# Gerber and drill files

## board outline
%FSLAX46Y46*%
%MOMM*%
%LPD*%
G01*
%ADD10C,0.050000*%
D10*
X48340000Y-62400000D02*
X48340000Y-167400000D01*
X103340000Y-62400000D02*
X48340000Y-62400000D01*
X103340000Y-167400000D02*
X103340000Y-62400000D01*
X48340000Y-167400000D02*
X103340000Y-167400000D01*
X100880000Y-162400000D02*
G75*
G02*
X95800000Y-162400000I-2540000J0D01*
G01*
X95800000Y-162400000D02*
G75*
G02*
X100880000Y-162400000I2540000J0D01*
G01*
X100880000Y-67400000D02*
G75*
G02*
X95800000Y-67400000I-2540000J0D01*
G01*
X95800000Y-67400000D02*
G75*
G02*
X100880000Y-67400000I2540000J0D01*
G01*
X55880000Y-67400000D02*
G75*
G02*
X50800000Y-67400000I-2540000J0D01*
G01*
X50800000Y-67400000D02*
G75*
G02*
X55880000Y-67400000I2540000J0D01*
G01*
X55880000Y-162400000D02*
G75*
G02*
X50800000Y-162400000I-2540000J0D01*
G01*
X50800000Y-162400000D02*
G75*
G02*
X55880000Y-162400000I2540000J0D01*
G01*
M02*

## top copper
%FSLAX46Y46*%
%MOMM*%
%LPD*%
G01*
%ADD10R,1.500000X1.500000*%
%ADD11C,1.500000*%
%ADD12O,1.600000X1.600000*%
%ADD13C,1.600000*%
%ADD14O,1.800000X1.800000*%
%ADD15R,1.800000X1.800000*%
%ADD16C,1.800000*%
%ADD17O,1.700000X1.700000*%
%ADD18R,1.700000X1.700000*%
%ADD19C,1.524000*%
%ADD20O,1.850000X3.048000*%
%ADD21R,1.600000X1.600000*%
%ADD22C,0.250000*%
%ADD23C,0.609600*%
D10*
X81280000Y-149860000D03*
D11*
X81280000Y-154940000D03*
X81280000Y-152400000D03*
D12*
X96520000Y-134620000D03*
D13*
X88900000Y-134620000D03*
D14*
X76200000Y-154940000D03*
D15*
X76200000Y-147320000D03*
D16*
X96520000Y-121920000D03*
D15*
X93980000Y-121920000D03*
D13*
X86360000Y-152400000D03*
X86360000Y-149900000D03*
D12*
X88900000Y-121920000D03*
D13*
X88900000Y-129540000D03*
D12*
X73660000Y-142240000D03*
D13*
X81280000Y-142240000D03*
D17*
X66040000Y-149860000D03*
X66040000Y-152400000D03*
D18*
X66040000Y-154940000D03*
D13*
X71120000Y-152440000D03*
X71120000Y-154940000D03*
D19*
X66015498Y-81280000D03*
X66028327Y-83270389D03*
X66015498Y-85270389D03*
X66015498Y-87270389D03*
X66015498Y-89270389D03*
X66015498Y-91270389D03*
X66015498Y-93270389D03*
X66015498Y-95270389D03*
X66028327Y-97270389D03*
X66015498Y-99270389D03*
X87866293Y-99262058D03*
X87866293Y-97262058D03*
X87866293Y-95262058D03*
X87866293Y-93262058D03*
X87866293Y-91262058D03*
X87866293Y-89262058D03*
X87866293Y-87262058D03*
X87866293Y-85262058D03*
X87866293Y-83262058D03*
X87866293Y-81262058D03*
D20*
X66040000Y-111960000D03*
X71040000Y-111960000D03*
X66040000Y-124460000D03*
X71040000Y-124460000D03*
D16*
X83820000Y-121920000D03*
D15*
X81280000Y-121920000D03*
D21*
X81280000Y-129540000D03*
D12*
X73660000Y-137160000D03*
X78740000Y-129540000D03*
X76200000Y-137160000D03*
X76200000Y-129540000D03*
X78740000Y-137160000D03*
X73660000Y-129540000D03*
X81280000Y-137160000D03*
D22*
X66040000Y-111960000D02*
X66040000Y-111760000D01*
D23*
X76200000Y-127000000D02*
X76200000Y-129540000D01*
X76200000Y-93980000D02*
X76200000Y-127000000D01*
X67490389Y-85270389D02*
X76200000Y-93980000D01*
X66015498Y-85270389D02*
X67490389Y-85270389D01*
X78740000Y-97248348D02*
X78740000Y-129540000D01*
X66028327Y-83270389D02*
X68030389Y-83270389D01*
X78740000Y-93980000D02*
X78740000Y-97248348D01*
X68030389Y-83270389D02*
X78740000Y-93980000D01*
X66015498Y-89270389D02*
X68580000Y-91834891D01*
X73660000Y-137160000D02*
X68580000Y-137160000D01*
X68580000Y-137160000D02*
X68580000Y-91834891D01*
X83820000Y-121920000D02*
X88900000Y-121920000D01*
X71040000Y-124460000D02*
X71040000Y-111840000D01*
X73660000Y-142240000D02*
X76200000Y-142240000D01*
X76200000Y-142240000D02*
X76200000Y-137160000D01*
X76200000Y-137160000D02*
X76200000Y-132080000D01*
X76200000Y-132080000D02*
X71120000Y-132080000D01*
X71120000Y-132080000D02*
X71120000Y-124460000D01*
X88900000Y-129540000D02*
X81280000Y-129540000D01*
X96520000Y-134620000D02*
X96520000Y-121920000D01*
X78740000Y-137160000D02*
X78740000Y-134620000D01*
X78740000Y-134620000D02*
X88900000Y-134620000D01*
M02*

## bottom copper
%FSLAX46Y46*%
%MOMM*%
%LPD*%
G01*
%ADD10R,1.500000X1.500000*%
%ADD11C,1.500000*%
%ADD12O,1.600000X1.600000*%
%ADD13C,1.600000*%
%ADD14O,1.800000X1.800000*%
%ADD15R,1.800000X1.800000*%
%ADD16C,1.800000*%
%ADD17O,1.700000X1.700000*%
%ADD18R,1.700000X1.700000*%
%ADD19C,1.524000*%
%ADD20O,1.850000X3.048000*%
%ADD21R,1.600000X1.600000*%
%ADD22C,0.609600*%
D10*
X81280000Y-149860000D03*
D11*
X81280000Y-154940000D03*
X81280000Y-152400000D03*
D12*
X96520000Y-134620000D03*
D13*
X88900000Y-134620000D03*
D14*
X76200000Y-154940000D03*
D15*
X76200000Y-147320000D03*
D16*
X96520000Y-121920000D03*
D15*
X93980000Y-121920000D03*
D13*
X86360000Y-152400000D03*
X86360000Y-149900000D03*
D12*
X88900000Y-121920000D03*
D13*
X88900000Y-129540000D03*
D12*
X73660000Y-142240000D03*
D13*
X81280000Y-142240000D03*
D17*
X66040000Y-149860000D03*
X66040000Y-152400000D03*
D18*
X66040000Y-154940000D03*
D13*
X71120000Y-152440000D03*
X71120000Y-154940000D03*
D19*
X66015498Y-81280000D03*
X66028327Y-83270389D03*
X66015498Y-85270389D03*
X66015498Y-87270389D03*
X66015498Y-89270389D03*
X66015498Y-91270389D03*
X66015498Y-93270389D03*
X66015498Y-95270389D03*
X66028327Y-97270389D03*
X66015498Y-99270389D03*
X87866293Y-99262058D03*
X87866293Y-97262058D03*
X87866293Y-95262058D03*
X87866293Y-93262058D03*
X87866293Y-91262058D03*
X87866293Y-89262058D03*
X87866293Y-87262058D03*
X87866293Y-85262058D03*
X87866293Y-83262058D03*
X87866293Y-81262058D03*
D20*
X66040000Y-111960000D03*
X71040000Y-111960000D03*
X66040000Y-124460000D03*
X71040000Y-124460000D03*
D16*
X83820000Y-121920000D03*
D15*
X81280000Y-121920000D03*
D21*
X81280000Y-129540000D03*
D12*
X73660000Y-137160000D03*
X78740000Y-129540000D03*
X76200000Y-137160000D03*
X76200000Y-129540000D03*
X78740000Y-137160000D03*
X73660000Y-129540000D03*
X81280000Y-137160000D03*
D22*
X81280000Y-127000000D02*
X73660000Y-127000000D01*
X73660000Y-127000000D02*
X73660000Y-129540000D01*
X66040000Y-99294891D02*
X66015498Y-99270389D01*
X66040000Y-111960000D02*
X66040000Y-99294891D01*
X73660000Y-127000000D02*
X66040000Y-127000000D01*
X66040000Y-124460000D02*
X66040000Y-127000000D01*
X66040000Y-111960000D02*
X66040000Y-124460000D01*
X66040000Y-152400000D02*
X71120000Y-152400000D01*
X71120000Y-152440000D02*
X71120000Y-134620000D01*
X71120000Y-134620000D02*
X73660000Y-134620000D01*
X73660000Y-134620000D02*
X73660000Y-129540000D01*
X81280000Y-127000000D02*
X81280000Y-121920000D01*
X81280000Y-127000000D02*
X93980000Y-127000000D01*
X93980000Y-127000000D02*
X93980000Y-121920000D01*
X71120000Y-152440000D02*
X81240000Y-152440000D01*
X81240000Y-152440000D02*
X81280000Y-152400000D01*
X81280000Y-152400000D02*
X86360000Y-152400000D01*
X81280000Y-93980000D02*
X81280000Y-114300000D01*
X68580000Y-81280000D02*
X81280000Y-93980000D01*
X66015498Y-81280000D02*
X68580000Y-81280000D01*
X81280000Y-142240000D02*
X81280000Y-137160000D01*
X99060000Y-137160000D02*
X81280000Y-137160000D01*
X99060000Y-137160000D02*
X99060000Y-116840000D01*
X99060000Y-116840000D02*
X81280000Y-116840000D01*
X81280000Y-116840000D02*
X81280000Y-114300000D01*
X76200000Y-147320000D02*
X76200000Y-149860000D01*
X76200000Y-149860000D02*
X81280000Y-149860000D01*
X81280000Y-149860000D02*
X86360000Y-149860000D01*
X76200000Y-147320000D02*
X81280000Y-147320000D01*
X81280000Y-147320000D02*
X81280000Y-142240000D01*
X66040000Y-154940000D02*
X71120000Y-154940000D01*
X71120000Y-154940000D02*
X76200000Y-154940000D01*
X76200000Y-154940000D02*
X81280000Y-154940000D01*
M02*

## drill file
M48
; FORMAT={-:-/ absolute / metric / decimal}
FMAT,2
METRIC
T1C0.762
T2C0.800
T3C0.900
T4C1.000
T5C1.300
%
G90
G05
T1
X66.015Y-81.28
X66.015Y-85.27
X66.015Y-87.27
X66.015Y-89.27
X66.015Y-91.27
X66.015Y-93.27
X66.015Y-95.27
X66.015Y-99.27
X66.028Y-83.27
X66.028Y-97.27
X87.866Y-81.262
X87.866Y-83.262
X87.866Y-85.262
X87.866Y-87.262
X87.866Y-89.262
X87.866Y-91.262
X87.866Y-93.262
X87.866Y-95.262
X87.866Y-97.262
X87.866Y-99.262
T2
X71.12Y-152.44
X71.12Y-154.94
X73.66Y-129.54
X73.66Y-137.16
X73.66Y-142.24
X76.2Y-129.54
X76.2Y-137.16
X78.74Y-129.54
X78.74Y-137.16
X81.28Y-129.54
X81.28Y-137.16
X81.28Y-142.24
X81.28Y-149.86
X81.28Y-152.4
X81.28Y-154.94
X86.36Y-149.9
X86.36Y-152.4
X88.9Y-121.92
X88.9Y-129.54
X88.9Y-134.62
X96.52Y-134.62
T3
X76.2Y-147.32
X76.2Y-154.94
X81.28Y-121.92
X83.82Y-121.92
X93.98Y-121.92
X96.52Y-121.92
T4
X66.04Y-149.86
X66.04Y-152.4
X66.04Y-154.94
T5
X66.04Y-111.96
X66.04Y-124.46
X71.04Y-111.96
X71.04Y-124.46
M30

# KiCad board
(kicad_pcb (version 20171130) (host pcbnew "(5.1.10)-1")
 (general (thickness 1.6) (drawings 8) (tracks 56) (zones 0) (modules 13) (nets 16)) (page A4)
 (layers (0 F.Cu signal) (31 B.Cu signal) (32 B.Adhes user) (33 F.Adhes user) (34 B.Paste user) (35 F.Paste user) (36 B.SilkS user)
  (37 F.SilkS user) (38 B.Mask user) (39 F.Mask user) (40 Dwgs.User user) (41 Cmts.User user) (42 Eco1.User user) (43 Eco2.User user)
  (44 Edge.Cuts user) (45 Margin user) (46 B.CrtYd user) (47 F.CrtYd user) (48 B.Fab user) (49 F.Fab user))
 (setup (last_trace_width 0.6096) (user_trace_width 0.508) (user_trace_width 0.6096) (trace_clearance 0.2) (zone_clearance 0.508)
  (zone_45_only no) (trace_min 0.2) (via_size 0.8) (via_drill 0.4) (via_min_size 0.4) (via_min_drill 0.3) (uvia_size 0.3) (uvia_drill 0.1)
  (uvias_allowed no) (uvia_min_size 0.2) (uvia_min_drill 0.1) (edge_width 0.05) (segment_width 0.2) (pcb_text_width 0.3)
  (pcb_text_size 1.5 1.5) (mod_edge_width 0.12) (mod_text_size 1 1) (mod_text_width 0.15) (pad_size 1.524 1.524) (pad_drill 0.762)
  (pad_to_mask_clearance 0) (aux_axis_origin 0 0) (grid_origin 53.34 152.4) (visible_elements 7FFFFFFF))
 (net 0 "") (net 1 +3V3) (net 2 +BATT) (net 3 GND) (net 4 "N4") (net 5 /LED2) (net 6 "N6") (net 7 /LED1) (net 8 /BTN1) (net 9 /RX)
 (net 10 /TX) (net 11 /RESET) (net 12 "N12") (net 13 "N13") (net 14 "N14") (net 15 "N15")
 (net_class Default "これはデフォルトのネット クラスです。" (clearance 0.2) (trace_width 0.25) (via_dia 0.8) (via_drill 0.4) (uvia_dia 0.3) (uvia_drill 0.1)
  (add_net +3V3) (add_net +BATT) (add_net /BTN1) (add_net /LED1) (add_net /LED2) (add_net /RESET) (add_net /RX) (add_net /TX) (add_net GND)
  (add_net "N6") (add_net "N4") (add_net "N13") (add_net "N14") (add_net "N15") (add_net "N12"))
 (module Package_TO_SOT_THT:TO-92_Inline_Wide (layer F.Cu) (at 81.28 149.86 270)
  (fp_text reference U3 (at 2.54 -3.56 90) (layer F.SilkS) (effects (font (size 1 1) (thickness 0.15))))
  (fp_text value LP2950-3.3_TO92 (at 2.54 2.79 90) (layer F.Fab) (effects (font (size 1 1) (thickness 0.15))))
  (pad 1 thru_hole rect (at 0 0 270) (size 1.5 1.5) (drill 0.8) (layers *.Cu *.Mask) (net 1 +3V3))
  (pad 3 thru_hole circle (at 5.08 0 270) (size 1.5 1.5) (drill 0.8) (layers *.Cu *.Mask) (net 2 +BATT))
  (pad 2 thru_hole circle (at 2.54 0 270) (size 1.5 1.5) (drill 0.8) (layers *.Cu *.Mask) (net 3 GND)))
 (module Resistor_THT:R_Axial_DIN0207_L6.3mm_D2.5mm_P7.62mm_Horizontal (layer F.Cu) (at 88.9 134.62)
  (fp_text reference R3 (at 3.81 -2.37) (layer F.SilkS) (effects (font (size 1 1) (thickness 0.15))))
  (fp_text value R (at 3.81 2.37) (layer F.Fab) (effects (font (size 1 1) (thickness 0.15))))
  (pad 2 thru_hole oval (at 7.62 0) (size 1.6 1.6) (drill 0.8) (layers *.Cu *.Mask) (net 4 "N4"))
  (pad 1 thru_hole circle (at 0 0) (size 1.6 1.6) (drill 0.8) (layers *.Cu *.Mask) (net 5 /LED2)))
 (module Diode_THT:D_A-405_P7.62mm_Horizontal (layer F.Cu) (at 76.2 147.32 270)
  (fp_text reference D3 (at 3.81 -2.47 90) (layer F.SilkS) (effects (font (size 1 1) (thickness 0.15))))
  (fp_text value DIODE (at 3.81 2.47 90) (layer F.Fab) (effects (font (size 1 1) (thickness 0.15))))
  (pad 2 thru_hole oval (at 7.62 0 270) (size 1.8 1.8) (drill 0.9) (layers *.Cu *.Mask) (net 2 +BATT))
  (pad 1 thru_hole rect (at 0 0 270) (size 1.8 1.8) (drill 0.9) (layers *.Cu *.Mask) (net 1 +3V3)))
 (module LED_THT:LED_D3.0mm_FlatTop (layer F.Cu) (at 93.98 121.92)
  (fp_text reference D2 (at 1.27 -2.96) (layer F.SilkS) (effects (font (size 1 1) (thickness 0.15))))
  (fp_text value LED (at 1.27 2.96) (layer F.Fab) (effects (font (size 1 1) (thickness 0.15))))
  (pad 2 thru_hole circle (at 2.54 0) (size 1.8 1.8) (drill 0.9) (layers *.Cu *.Mask) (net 4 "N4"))
  (pad 1 thru_hole rect (at 0 0) (size 1.8 1.8) (drill 0.9) (layers *.Cu *.Mask) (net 3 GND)))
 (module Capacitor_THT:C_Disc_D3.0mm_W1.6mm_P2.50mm (layer F.Cu) (at 86.36 149.9 270)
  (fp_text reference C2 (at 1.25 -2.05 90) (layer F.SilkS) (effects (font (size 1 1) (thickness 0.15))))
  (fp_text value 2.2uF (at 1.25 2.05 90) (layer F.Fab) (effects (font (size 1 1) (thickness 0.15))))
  (pad 2 thru_hole circle (at 2.5 0 270) (size 1.6 1.6) (drill 0.8) (layers *.Cu *.Mask) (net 3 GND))
  (pad 1 thru_hole circle (at 0 0 270) (size 1.6 1.6) (drill 0.8) (layers *.Cu *.Mask) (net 1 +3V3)))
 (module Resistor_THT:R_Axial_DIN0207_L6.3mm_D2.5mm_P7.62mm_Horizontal (layer F.Cu) (at 88.9 129.54 90)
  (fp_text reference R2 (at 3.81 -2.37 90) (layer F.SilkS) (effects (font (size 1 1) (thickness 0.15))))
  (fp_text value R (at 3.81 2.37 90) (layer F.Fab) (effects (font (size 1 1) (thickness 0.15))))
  (pad 2 thru_hole oval (at 7.62 0 90) (size 1.6 1.6) (drill 0.8) (layers *.Cu *.Mask) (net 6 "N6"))
  (pad 1 thru_hole circle (at 0 0 90) (size 1.6 1.6) (drill 0.8) (layers *.Cu *.Mask) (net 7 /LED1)))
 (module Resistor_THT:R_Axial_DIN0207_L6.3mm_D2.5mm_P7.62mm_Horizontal (layer F.Cu) (at 81.28 142.24 180)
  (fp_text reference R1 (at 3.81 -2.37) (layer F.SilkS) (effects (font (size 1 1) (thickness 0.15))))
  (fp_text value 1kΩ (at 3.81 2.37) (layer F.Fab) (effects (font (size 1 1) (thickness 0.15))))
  (pad 2 thru_hole oval (at 7.62 0 180) (size 1.6 1.6) (drill 0.8) (layers *.Cu *.Mask) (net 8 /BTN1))
  (pad 1 thru_hole circle (at 0 0 180) (size 1.6 1.6) (drill 0.8) (layers *.Cu *.Mask) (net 1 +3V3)))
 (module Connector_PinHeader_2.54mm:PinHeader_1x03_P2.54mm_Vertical (layer F.Cu) (at 66.04 154.94 180)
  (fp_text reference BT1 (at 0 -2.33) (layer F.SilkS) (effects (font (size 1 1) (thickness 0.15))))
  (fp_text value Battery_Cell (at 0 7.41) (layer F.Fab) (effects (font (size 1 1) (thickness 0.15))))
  (pad 3 thru_hole oval (at 0 5.08 180) (size 1.7 1.7) (drill 1) (layers *.Cu *.Mask))
  (pad 2 thru_hole oval (at 0 2.54 180) (size 1.7 1.7) (drill 1) (layers *.Cu *.Mask) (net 3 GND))
  (pad 1 thru_hole rect (at 0 0 180) (size 1.7 1.7) (drill 1) (layers *.Cu *.Mask) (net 2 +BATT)))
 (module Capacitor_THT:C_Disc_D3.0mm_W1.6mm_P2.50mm (layer F.Cu) (at 71.12 154.94 90)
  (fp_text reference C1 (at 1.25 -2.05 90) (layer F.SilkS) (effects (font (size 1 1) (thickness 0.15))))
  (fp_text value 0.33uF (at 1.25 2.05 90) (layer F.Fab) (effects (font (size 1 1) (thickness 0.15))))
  (pad 2 thru_hole circle (at 2.5 0 90) (size 1.6 1.6) (drill 0.8) (layers *.Cu *.Mask) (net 3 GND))
  (pad 1 thru_hole circle (at 0 0 90) (size 1.6 1.6) (drill 0.8) (layers *.Cu *.Mask) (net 2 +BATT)))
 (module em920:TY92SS (layer F.Cu) (at 64.77 107.929212)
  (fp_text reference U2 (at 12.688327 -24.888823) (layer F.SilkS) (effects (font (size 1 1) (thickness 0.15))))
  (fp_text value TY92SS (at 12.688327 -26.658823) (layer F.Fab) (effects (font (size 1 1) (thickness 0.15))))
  (pad 1 thru_hole circle (at 1.245498 -26.649212) (size 1.524 1.524) (drill 0.762) (layers *.Cu *.Mask) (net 1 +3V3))
  (pad 2 thru_hole circle (at 1.258327 -24.658823) (size 1.524 1.524) (drill 0.762) (layers *.Cu *.Mask) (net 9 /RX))
  (pad 3 thru_hole circle (at 1.245498 -22.658823) (size 1.524 1.524) (drill 0.762) (layers *.Cu *.Mask) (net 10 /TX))
  (pad 4 thru_hole circle (at 1.245498 -20.658823) (size 1.524 1.524) (drill 0.762) (layers *.Cu *.Mask))
  (pad 5 thru_hole circle (at 1.245498 -18.658823) (size 1.524 1.524) (drill 0.762) (layers *.Cu *.Mask) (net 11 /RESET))
  (pad 6 thru_hole circle (at 1.245498 -16.658823) (size 1.524 1.524) (drill 0.762) (layers *.Cu *.Mask))
  (pad 7 thru_hole circle (at 1.245498 -14.658823) (size 1.524 1.524) (drill 0.762) (layers *.Cu *.Mask))
  (pad 8 thru_hole circle (at 1.245498 -12.658823) (size 1.524 1.524) (drill 0.762) (layers *.Cu *.Mask))
  (pad 9 thru_hole circle (at 1.258327 -10.658823) (size 1.524 1.524) (drill 0.762) (layers *.Cu *.Mask) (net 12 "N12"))
  (pad 10 thru_hole circle (at 1.245498 -8.658823) (size 1.524 1.524) (drill 0.762) (layers *.Cu *.Mask) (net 3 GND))
  (pad 11 thru_hole circle (at 23.096293 -8.667154) (size 1.524 1.524) (drill 0.762) (layers *.Cu *.Mask))
  (pad 12 thru_hole circle (at 23.096293 -10.667154) (size 1.524 1.524) (drill 0.762) (layers *.Cu *.Mask) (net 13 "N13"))
  (pad 13 thru_hole circle (at 23.096293 -12.667154) (size 1.524 1.524) (drill 0.762) (layers *.Cu *.Mask) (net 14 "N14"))
  (pad 14 thru_hole circle (at 23.096293 -14.667154) (size 1.524 1.524) (drill 0.762) (layers *.Cu *.Mask))
  (pad 15 thru_hole circle (at 23.096293 -16.667154) (size 1.524 1.524) (drill 0.762) (layers *.Cu *.Mask))
  (pad 16 thru_hole circle (at 23.096293 -18.667154) (size 1.524 1.524) (drill 0.762) (layers *.Cu *.Mask) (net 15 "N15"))
  (pad 17 thru_hole circle (at 23.096293 -20.667154) (size 1.524 1.524) (drill 0.762) (layers *.Cu *.Mask))
  (pad 18 thru_hole circle (at 23.096293 -22.667154) (size 1.524 1.524) (drill 0.762) (layers *.Cu *.Mask))
  (pad 19 thru_hole circle (at 23.096293 -24.667154) (size 1.524 1.524) (drill 0.762) (layers *.Cu *.Mask))
  (pad 20 thru_hole circle (at 23.096293 -26.667154) (size 1.524 1.524) (drill 0.762) (layers *.Cu *.Mask)))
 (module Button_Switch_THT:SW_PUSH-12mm (layer F.Cu) (at 71.04 111.96 270)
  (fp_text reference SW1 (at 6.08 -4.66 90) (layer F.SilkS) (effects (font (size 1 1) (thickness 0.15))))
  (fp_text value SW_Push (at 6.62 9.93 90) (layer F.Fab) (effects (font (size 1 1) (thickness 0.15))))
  (pad 2 thru_hole oval (at 0 5 270) (size 3.048 1.85) (drill 1.3) (layers *.Cu *.Mask) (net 3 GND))
  (pad 1 thru_hole oval (at 0 0 270) (size 3.048 1.85) (drill 1.3) (layers *.Cu *.Mask) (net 8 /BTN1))
  (pad 2 thru_hole oval (at 12.5 5 270) (size 3.048 1.85) (drill 1.3) (layers *.Cu *.Mask) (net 3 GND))
  (pad 1 thru_hole oval (at 12.5 0 270) (size 3.048 1.85) (drill 1.3) (layers *.Cu *.Mask) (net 8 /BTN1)))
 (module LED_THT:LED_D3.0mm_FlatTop (layer F.Cu) (at 81.28 121.92)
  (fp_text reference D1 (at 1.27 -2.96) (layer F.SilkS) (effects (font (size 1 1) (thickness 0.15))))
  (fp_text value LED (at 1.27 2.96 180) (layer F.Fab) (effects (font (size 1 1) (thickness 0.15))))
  (pad 2 thru_hole circle (at 2.54 0) (size 1.8 1.8) (drill 0.9) (layers *.Cu *.Mask) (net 6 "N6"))
  (pad 1 thru_hole rect (at 0 0) (size 1.8 1.8) (drill 0.9) (layers *.Cu *.Mask) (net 3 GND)))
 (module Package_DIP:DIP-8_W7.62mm (layer F.Cu) (at 81.28 129.54 270)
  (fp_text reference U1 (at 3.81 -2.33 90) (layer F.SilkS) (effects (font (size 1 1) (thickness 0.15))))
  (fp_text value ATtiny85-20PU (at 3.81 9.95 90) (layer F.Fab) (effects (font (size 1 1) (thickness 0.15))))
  (pad 1 thru_hole rect (at 0 0 270) (size 1.6 1.6) (drill 0.8) (layers *.Cu *.Mask) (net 7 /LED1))
  (pad 5 thru_hole oval (at 7.62 7.62 270) (size 1.6 1.6) (drill 0.8) (layers *.Cu *.Mask) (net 11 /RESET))
  (pad 2 thru_hole oval (at 0 2.54 270) (size 1.6 1.6) (drill 0.8) (layers *.Cu *.Mask) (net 9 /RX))
  (pad 6 thru_hole oval (at 7.62 5.08 270) (size 1.6 1.6) (drill 0.8) (layers *.Cu *.Mask) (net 8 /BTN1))
  (pad 3 thru_hole oval (at 0 5.08 270) (size 1.6 1.6) (drill 0.8) (layers *.Cu *.Mask) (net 10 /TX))
  (pad 7 thru_hole oval (at 7.62 2.54 270) (size 1.6 1.6) (drill 0.8) (layers *.Cu *.Mask) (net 5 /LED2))
  (pad 4 thru_hole oval (at 0 7.62 270) (size 1.6 1.6) (drill 0.8) (layers *.Cu *.Mask) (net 3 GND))
  (pad 8 thru_hole oval (at 7.62 0 270) (size 1.6 1.6) (drill 0.8) (layers *.Cu *.Mask) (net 1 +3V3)))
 (gr_line (start 48.34 62.4) (end 48.34 167.4) (layer Edge.Cuts) (width 0.05))
 (gr_line (start 103.34 62.4) (end 48.34 62.4) (layer Edge.Cuts) (width 0.05))
 (gr_line (start 103.34 167.4) (end 103.34 62.4) (layer Edge.Cuts) (width 0.05))
 (gr_line (start 48.34 167.4) (end 103.34 167.4) (layer Edge.Cuts) (width 0.05))
 (gr_circle (center 98.34 162.4) (end 98.34 159.86) (layer Edge.Cuts) (width 0.05))
 (gr_circle (center 98.34 67.4) (end 98.34 69.94) (layer Edge.Cuts) (width 0.05))
 (gr_circle (center 53.34 67.4) (end 53.34 69.94) (layer Edge.Cuts) (width 0.05))
 (gr_circle (center 53.34 162.4) (end 55.88 162.4) (layer Edge.Cuts) (width 0.05))
 (segment (start 81.28 127) (end 73.66 127) (width 0.6096) (layer B.Cu) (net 3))
 (segment (start 73.66 127) (end 73.66 129.54) (width 0.6096) (layer B.Cu) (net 3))
 (segment (start 66.04 99.294891) (end 66.015498 99.270389) (width 0.6096) (layer B.Cu) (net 3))
 (segment (start 66.04 111.96) (end 66.04 99.294891) (width 0.6096) (layer B.Cu) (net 3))
 (segment (start 73.66 127) (end 66.04 127) (width 0.6096) (layer B.Cu) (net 3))
 (segment (start 66.04 124.46) (end 66.04 127) (width 0.6096) (layer B.Cu) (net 3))
 (segment (start 66.04 111.96) (end 66.04 111.76) (width 0.25) (layer F.Cu) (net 3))
 (segment (start 66.04 111.96) (end 66.04 124.46) (width 0.6096) (layer B.Cu) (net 3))
 (segment (start 66.04 152.4) (end 71.12 152.4) (width 0.6096) (layer B.Cu) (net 3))
 (segment (start 71.12 152.44) (end 71.12 134.62) (width 0.6096) (layer B.Cu) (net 3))
 (segment (start 71.12 134.62) (end 73.66 134.62) (width 0.6096) (layer B.Cu) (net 3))
 (segment (start 73.66 134.62) (end 73.66 129.54) (width 0.6096) (layer B.Cu) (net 3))
 (segment (start 81.28 127) (end 81.28 121.92) (width 0.6096) (layer B.Cu) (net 3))
 (segment (start 81.28 127) (end 93.98 127) (width 0.6096) (layer B.Cu) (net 3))
 (segment (start 93.98 127) (end 93.98 121.92) (width 0.6096) (layer B.Cu) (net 3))
 (segment (start 71.12 152.44) (end 81.24 152.44) (width 0.6096) (layer B.Cu) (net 3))
 (segment (start 81.24 152.44) (end 81.28 152.4) (width 0.6096) (layer B.Cu) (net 3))
 (segment (start 81.28 152.4) (end 86.36 152.4) (width 0.6096) (layer B.Cu) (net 3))
 (segment (start 81.28 93.98) (end 81.28 114.3) (width 0.6096) (layer B.Cu) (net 1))
 (segment (start 68.58 81.28) (end 81.28 93.98) (width 0.6096) (layer B.Cu) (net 1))
 (segment (start 66.015498 81.28) (end 68.58 81.28) (width 0.6096) (layer B.Cu) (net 1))
 (segment (start 81.28 142.24) (end 81.28 137.16) (width 0.6096) (layer B.Cu) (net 1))
 (segment (start 99.06 137.16) (end 81.28 137.16) (width 0.6096) (layer B.Cu) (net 1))
 (segment (start 99.06 137.16) (end 99.06 116.84) (width 0.6096) (layer B.Cu) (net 1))
 (segment (start 99.06 116.84) (end 81.28 116.84) (width 0.6096) (layer B.Cu) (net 1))
 (segment (start 81.28 116.84) (end 81.28 114.3) (width 0.6096) (layer B.Cu) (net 1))
 (segment (start 76.2 147.32) (end 76.2 149.86) (width 0.6096) (layer B.Cu) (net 1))
 (segment (start 76.2 149.86) (end 81.28 149.86) (width 0.6096) (layer B.Cu) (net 1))
 (segment (start 81.28 149.86) (end 86.36 149.86) (width 0.6096) (layer B.Cu) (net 1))
 (segment (start 76.2 147.32) (end 81.28 147.32) (width 0.6096) (layer B.Cu) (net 1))
 (segment (start 81.28 147.32) (end 81.28 142.24) (width 0.6096) (layer B.Cu) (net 1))
 (segment (start 76.2 127) (end 76.2 129.54) (width 0.6096) (layer F.Cu) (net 10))
 (segment (start 76.2 93.98) (end 76.2 127) (width 0.6096) (layer F.Cu) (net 10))
 (segment (start 67.490389 85.270389) (end 76.2 93.98) (width 0.6096) (layer F.Cu) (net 10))
 (segment (start 66.015498 85.270389) (end 67.490389 85.270389) (width 0.6096) (layer F.Cu) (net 10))
 (segment (start 78.74 97.248348) (end 78.74 129.54) (width 0.6096) (layer F.Cu) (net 9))
 (segment (start 66.028327 83.270389) (end 68.030389 83.270389) (width 0.6096) (layer F.Cu) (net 9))
 (segment (start 78.74 93.98) (end 78.74 97.248348) (width 0.6096) (layer F.Cu) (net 9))
 (segment (start 68.030389 83.270389) (end 78.74 93.98) (width 0.6096) (layer F.Cu) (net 9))
 (segment (start 66.015498 89.270389) (end 68.58 91.834891) (width 0.6096) (layer F.Cu) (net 11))
 (segment (start 73.66 137.16) (end 68.58 137.16) (width 0.6096) (layer F.Cu) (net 11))
 (segment (start 68.58 137.16) (end 68.58 91.834891) (width 0.6096) (layer F.Cu) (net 11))
 (segment (start 66.04 154.94) (end 71.12 154.94) (width 0.6096) (layer B.Cu) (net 2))
 (segment (start 71.12 154.94) (end 76.2 154.94) (width 0.6096) (layer B.Cu) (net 2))
 (segment (start 76.2 154.94) (end 81.28 154.94) (width 0.6096) (layer B.Cu) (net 2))
 (segment (start 83.82 121.92) (end 88.9 121.92) (width 0.6096) (layer F.Cu) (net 6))
 (segment (start 71.04 124.46) (end 71.04 111.84) (width 0.6096) (layer F.Cu) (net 8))
 (segment (start 73.66 142.24) (end 76.2 142.24) (width 0.6096) (layer F.Cu) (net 8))
 (segment (start 76.2 142.24) (end 76.2 137.16) (width 0.6096) (layer F.Cu) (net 8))
 (segment (start 76.2 137.16) (end 76.2 132.08) (width 0.6096) (layer F.Cu) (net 8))
 (segment (start 76.2 132.08) (end 71.12 132.08) (width 0.6096) (layer F.Cu) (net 8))
 (segment (start 71.12 132.08) (end 71.12 124.46) (width 0.6096) (layer F.Cu) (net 8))
 (segment (start 88.9 129.54) (end 81.28 129.54) (width 0.6096) (layer F.Cu) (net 7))
 (segment (start 96.52 134.62) (end 96.52 121.92) (width 0.6096) (layer F.Cu) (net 4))
 (segment (start 78.74 137.16) (end 78.74 134.62) (width 0.6096) (layer F.Cu) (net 5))
 (segment (start 78.74 134.62) (end 88.9 134.62) (width 0.6096) (layer F.Cu) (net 5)))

